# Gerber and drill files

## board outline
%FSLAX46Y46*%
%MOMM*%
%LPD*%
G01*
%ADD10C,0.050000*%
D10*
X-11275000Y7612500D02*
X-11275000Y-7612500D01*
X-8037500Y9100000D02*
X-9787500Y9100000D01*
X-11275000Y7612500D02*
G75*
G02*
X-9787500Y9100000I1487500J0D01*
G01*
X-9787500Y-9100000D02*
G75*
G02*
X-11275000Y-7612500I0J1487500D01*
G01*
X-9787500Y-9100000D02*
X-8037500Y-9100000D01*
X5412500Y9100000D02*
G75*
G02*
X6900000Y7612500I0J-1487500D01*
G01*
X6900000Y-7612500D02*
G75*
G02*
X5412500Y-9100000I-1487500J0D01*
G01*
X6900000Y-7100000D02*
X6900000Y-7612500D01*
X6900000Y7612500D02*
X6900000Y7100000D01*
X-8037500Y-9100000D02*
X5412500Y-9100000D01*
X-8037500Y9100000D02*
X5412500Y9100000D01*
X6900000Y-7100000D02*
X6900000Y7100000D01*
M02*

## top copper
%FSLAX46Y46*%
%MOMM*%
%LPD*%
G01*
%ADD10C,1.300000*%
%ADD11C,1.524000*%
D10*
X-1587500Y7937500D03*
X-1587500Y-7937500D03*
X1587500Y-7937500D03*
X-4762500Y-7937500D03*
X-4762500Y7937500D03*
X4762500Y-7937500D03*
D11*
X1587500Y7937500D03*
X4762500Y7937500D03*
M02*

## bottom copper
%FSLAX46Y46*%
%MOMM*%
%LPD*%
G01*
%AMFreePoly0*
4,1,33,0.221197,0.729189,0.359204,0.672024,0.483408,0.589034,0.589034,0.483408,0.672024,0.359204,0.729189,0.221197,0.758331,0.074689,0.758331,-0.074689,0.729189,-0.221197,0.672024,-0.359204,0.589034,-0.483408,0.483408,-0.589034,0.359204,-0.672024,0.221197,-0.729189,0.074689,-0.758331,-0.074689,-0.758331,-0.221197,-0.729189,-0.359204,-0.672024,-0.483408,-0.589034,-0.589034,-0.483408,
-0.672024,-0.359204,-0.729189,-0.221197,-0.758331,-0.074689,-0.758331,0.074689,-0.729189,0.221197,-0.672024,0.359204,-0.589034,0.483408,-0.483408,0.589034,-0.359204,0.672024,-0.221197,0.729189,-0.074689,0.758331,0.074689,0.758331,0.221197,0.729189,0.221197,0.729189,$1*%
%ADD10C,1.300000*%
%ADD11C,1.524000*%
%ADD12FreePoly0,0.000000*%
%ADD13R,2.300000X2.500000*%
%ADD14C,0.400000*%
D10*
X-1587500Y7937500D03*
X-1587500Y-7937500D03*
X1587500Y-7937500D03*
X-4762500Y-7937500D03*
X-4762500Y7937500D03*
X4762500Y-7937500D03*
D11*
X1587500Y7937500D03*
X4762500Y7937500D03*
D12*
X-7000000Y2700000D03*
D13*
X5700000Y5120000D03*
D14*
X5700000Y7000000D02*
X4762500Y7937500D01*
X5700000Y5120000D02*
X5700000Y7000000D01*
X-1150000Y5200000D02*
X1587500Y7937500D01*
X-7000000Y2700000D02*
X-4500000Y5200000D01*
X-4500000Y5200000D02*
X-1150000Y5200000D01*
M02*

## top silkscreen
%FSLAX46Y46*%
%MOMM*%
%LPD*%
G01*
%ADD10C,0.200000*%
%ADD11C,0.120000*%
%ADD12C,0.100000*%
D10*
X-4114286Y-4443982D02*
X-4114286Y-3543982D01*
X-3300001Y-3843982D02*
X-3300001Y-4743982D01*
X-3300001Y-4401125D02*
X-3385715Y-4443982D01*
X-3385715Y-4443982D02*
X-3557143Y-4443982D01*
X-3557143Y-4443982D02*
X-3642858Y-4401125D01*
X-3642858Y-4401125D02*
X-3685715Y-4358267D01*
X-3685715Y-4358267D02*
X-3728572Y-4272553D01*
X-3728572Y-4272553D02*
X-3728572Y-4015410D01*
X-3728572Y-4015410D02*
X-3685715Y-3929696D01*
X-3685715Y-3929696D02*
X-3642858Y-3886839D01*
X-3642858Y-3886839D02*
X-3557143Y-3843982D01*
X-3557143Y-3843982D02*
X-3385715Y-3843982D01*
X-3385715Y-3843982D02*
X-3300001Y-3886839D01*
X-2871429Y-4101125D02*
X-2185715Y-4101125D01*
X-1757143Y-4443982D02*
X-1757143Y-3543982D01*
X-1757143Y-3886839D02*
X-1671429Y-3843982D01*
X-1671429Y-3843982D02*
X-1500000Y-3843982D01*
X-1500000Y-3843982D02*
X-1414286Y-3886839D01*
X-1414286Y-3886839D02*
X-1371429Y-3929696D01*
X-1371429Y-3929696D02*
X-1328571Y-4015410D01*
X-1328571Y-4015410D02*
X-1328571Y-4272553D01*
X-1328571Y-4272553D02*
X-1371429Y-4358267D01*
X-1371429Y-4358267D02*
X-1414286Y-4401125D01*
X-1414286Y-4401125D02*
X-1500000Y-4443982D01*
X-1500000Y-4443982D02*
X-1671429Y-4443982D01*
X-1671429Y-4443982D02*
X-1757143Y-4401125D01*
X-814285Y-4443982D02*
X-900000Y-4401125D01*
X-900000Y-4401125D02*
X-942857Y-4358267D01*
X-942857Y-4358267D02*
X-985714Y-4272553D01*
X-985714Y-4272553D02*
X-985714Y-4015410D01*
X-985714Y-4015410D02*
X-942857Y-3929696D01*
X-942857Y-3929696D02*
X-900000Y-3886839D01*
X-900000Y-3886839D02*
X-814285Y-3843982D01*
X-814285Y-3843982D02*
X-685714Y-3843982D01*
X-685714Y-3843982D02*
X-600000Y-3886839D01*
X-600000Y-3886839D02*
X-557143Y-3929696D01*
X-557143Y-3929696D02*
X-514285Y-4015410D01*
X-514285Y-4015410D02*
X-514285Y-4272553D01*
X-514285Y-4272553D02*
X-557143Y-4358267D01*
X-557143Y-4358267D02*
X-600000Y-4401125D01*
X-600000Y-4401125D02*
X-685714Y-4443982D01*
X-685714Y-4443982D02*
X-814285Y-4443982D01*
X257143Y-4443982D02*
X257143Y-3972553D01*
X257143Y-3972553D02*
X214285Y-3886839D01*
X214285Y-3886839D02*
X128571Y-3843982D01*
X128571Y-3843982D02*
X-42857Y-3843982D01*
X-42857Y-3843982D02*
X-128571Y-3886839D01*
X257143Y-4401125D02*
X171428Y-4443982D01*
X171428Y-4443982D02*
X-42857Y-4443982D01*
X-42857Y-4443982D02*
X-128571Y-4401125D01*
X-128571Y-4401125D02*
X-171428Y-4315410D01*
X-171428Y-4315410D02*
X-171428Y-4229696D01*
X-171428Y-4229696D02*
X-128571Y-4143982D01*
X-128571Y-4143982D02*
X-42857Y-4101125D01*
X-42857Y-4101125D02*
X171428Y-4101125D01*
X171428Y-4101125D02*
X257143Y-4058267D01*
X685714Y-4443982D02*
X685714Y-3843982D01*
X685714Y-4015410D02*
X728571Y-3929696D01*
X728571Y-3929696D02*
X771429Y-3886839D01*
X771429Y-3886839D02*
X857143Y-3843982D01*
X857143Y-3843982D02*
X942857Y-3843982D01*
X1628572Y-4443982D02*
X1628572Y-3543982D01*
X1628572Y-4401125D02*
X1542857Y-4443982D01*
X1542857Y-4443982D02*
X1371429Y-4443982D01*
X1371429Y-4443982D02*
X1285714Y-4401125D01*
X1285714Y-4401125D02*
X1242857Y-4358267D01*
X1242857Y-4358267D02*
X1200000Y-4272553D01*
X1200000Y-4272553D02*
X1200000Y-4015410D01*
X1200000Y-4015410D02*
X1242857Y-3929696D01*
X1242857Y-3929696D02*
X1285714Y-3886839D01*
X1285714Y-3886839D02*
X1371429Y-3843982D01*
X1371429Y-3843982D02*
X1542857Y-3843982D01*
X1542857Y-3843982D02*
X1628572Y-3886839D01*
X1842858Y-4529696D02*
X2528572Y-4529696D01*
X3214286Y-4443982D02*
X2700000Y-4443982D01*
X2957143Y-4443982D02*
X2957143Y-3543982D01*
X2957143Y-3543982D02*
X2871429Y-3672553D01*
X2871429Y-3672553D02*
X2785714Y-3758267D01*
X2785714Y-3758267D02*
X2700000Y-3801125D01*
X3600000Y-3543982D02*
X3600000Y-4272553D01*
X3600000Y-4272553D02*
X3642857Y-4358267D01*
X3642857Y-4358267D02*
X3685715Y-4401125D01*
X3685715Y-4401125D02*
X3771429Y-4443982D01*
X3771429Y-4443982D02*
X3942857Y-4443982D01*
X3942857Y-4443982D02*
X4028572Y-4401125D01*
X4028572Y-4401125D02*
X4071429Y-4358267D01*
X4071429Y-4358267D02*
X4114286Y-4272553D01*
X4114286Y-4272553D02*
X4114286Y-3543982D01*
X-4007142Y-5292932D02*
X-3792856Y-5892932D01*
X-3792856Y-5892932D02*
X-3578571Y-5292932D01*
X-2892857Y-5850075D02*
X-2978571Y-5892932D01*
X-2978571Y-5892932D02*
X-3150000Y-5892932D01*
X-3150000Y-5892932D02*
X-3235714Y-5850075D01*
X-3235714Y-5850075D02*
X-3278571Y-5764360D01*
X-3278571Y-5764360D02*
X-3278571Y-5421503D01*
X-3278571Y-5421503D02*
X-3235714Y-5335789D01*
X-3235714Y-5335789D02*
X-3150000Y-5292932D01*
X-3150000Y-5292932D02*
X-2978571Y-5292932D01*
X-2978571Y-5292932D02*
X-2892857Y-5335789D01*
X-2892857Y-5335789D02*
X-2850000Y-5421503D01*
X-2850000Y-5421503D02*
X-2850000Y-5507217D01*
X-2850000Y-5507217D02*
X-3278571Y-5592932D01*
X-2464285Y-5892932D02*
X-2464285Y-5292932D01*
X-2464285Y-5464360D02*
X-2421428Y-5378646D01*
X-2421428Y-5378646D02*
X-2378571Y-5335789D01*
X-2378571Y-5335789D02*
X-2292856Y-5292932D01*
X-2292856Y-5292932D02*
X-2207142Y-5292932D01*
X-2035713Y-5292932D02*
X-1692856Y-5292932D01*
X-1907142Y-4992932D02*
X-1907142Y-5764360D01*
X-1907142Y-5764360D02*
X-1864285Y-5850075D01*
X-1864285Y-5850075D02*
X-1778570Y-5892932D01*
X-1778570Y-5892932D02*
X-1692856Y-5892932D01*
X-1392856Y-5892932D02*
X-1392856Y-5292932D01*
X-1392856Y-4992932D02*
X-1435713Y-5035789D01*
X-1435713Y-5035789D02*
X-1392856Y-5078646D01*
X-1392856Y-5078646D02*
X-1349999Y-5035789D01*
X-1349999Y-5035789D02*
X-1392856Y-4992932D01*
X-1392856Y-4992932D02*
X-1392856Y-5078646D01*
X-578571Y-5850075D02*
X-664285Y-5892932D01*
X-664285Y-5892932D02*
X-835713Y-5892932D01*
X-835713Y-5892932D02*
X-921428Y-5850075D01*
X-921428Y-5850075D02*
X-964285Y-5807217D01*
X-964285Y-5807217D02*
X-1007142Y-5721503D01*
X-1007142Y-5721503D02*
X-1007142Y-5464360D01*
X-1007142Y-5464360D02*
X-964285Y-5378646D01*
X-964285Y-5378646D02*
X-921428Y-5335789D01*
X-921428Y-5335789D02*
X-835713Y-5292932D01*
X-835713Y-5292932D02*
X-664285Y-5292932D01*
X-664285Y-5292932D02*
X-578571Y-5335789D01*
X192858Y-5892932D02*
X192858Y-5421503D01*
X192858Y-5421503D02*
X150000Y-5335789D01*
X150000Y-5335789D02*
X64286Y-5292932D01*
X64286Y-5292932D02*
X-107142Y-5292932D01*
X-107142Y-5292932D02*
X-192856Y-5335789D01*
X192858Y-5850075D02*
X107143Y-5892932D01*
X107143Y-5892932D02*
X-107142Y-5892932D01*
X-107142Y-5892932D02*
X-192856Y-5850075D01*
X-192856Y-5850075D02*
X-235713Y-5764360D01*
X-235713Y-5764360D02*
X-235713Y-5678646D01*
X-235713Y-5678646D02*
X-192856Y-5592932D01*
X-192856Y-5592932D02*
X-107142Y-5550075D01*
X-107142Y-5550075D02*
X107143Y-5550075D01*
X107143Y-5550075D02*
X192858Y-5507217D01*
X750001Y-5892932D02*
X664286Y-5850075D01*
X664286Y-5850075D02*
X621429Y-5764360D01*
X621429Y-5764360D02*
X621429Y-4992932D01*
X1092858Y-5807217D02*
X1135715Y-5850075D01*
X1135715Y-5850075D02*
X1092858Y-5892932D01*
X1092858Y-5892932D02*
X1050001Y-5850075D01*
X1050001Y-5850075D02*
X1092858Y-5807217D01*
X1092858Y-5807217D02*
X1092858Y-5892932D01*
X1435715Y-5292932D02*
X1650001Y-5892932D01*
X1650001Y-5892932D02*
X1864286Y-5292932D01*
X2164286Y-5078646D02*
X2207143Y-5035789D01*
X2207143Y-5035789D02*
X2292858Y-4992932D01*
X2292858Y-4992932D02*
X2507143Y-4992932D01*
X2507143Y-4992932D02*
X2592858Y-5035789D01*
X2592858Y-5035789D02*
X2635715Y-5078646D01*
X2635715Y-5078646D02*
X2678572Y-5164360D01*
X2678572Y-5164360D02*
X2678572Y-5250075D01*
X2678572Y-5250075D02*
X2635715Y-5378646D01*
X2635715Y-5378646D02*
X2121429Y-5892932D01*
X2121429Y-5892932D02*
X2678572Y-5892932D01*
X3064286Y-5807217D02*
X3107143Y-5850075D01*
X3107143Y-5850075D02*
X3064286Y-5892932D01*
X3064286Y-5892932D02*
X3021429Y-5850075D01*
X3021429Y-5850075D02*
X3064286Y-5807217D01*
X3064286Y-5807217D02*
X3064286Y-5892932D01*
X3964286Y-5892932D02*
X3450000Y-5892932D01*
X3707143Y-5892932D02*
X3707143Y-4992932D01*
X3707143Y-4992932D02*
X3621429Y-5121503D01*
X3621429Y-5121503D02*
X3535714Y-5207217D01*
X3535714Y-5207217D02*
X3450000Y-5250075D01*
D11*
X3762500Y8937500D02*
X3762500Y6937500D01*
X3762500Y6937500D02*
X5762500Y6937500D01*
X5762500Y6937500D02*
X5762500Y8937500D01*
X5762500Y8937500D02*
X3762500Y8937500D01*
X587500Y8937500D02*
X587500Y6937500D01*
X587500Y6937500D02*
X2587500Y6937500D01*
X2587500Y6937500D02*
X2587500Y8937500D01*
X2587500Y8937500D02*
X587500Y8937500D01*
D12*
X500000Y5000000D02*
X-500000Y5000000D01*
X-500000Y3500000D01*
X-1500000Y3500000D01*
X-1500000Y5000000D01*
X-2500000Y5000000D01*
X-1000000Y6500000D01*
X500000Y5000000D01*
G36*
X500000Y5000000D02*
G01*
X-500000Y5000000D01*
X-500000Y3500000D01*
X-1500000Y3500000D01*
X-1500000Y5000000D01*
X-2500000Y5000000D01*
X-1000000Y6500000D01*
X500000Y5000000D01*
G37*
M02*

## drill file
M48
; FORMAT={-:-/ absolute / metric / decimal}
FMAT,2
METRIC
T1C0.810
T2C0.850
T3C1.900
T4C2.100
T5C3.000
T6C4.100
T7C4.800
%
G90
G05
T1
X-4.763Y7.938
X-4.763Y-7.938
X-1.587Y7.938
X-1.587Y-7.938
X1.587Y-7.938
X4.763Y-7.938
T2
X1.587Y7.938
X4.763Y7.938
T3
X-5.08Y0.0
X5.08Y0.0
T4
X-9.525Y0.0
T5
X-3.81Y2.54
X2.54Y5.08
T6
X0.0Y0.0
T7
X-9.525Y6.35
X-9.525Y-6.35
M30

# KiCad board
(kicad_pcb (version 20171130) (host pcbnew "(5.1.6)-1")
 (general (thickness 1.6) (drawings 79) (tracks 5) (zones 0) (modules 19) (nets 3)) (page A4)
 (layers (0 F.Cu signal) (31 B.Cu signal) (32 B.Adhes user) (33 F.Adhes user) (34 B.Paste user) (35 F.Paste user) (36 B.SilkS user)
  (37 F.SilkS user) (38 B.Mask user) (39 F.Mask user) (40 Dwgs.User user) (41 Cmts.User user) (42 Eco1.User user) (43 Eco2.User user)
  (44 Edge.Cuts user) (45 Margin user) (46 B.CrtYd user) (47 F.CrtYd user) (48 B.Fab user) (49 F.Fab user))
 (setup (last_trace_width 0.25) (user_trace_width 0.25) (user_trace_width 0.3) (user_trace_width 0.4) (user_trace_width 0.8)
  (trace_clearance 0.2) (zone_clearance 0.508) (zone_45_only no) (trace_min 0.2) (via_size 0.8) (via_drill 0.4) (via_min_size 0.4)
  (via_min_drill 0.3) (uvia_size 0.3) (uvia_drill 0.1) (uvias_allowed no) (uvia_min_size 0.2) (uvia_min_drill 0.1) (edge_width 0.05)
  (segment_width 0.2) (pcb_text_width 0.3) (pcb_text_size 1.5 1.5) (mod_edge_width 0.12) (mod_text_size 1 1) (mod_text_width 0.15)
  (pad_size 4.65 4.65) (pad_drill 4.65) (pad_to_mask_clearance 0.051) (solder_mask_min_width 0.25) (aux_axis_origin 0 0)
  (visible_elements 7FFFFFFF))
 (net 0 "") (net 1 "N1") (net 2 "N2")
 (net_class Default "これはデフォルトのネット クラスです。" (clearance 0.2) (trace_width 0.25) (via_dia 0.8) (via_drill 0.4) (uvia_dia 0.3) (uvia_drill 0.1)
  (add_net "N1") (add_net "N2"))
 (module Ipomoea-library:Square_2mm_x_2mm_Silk (layer F.Cu) (at 4.7625 -7.9375)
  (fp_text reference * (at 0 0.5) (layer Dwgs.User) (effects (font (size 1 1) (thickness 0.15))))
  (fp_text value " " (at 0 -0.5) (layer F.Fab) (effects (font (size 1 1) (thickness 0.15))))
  (fp_line (start -1 -1) (end -1 1) (layer F.SilkS) (width 0.12))
  (fp_line (start -1 1) (end 1 1) (layer F.SilkS) (width 0.12))
  (fp_line (start 1 1) (end 1 -1) (layer F.SilkS) (width 0.12))
  (fp_line (start 1 -1) (end -1 -1) (layer F.SilkS) (width 0.12)))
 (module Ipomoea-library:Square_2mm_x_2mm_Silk (layer F.Cu) (at 1.5875 -7.9375)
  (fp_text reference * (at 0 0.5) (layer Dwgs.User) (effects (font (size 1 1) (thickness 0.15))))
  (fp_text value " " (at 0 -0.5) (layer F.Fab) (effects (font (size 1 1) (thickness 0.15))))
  (fp_line (start -1 -1) (end -1 1) (layer F.SilkS) (width 0.12))
  (fp_line (start -1 1) (end 1 1) (layer F.SilkS) (width 0.12))
  (fp_line (start 1 1) (end 1 -1) (layer F.SilkS) (width 0.12))
  (fp_line (start 1 -1) (end -1 -1) (layer F.SilkS) (width 0.12)))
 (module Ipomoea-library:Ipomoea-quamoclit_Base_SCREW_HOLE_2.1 (layer F.Cu) (at -9.525 0)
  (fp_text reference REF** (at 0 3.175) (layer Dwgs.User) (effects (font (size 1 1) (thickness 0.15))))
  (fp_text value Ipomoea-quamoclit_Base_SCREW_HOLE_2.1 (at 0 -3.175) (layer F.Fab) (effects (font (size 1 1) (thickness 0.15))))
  (pad "" np_thru_hole circle (at 0 0) (size 2.1 2.1) (drill 2.1) (layers *.Cu *.Mask)))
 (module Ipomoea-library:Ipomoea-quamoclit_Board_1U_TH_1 (layer F.Cu) (at -1.5875 -7.9375)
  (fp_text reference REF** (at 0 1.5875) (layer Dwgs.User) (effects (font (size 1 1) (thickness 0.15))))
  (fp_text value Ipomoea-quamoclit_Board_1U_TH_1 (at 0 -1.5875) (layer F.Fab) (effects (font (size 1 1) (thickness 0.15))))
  (pad "" thru_hole circle (at 0 0 180) (size 1.3 1.3) (drill 0.81) (layers *.Cu *.Mask)))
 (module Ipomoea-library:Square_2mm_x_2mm (layer F.Cu) (at -1.5875 -7.9375)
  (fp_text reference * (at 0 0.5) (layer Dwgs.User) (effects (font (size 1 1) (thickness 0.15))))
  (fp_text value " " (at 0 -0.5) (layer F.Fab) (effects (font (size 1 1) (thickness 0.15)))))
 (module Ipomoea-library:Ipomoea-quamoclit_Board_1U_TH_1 (layer F.Cu) (at -1.5875 7.9375)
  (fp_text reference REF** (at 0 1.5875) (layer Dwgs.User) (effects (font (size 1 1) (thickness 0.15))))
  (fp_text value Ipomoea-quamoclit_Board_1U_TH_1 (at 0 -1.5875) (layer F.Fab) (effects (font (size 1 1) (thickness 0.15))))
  (pad "" thru_hole circle (at 0 0 180) (size 1.3 1.3) (drill 0.81) (layers *.Cu *.Mask)))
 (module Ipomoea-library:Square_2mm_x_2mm (layer F.Cu) (at -1.5875 7.9375)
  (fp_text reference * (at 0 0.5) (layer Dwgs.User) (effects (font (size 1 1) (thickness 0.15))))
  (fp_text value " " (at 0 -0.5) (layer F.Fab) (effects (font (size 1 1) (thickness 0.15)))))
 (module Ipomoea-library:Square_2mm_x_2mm (layer F.Cu) (at 1.5875 7.9375)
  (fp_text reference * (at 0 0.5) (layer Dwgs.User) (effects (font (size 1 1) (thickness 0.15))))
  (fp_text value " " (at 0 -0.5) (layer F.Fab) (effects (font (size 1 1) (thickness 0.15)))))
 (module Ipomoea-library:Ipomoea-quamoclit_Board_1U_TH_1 (layer F.Cu) (at 1.5875 7.9375)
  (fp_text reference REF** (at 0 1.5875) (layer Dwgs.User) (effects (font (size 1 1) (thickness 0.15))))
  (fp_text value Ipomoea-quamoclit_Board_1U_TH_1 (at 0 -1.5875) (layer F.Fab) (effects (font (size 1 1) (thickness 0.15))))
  (pad "" thru_hole circle (at 0 0 180) (size 1.3 1.3) (drill 0.81) (layers *.Cu *.Mask)))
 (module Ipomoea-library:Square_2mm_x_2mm (layer F.Cu) (at 4.7625 7.9375)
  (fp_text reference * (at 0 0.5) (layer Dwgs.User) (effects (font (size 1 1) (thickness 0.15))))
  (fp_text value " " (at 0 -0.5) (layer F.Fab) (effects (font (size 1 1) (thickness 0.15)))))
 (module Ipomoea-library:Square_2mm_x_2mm (layer F.Cu) (at -4.7625 7.9375)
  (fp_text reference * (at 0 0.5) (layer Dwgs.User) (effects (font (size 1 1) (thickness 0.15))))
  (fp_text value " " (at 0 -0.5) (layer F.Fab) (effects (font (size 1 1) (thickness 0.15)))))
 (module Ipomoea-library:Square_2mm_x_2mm (layer F.Cu) (at -4.7625 -7.9375)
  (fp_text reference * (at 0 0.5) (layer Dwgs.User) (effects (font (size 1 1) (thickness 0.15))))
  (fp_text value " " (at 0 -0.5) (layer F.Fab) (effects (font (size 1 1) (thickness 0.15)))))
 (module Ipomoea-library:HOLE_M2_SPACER (layer F.Cu) (at -9.525 6.35)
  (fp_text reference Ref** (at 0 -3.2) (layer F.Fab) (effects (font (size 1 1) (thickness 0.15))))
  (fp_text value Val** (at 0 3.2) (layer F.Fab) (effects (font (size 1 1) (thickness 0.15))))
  (pad "" np_thru_hole circle (at 0 0) (size 4.8 4.8) (drill 4.8) (layers *.Cu *.Mask)))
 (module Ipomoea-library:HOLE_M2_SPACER (layer F.Cu) (at -9.525 -6.35)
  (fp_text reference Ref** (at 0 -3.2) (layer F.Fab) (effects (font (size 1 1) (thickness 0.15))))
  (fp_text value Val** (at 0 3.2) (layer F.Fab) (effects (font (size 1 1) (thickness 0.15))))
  (pad "" np_thru_hole circle (at 0 0) (size 4.8 4.8) (drill 4.8) (layers *.Cu *.Mask)))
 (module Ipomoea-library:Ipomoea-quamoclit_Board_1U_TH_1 (layer F.Cu) (at -4.7625 7.9375)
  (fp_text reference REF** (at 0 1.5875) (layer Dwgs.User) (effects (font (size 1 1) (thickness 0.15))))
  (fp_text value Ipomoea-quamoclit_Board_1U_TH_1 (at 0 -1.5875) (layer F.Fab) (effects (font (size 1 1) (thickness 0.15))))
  (pad "" thru_hole circle (at 0 0 180) (size 1.3 1.3) (drill 0.81) (layers *.Cu *.Mask)))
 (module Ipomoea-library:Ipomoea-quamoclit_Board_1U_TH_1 (layer F.Cu) (at -4.7625 -7.9375)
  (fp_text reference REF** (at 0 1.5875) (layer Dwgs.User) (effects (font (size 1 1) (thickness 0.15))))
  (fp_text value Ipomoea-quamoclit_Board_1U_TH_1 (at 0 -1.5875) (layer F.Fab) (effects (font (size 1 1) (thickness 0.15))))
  (pad "" thru_hole circle (at 0 0 180) (size 1.3 1.3) (drill 0.81) (layers *.Cu *.Mask)))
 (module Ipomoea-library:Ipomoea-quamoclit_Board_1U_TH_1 (layer F.Cu) (at 4.7625 7.9375)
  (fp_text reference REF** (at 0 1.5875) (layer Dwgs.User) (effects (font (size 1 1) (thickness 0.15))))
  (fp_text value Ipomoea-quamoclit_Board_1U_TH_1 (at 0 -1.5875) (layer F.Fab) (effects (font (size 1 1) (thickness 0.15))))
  (pad "" thru_hole circle (at 0 0 180) (size 1.3 1.3) (drill 0.81) (layers *.Cu *.Mask)))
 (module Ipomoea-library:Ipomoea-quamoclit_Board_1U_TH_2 (layer F.Cu) (at 3.175 -7.9375)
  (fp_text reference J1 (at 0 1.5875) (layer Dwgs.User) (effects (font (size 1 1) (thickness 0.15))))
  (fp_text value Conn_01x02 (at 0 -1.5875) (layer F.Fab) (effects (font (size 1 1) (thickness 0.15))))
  (pad 1 thru_hole circle (at -1.5875 0 180) (size 1.524 1.524) (drill 0.85) (layers *.Cu *.Mask) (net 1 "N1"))
  (pad 2 thru_hole circle (at 1.5875 0 180) (size 1.524 1.524) (drill 0.85) (layers *.Cu *.Mask) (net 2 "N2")))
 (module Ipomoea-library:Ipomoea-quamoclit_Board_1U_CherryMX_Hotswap (layer F.Cu) (at 0 0)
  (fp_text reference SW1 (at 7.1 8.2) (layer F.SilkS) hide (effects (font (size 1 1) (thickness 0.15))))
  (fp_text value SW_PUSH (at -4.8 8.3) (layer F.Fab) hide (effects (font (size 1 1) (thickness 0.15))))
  (fp_poly (pts (xy 0.5 -5) (xy -0.5 -5) (xy -0.5 -3.5) (xy -1.5 -3.5) (xy -1.5 -5) (xy -2.5 -5) (xy -1 -6.5)) (layer F.SilkS) (width 0.1))
  (pad "" np_thru_hole circle (at 0 0 90) (size 4.1 4.1) (drill 4.1) (layers *.Cu *.Mask))
  (pad "" np_thru_hole circle (at 5.08 0) (size 1.9 1.9) (drill 1.9) (layers *.Cu *.Mask))
  (pad "" np_thru_hole circle (at -5.08 0) (size 1.9 1.9) (drill 1.9) (layers *.Cu *.Mask))
  (pad 1 smd custom (at -7 -2.7) (size 1.524 1.524) (layers B.Cu B.Paste B.Mask) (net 1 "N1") (zone_connect 0)
   (options (clearance outline) (anchor circle)) (primitives))
  (pad "" np_thru_hole circle (at 2.54 -5.08 180) (size 3 3) (drill 3) (layers *.Cu *.Mask))
  (pad 2 smd rect (at 5.7 -5.12 180) (size 2.3 2.5) (layers B.Cu B.Paste B.Mask) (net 2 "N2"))
  (pad "" np_thru_hole circle (at -3.81 -2.54 180) (size 3 3) (drill 3) (layers *.Cu *.Mask)))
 (gr_line (start -11.275 -7.6125) (end -11.275 7.6125) (layer Edge.Cuts) (width 0.05))
 (gr_line (start -8.0375 -9.1) (end -9.7875 -9.1) (layer Edge.Cuts) (width 0.05))
 (gr_arc (start -9.7875 -7.6125) (end -9.7875 -9.1) (angle -90) (layer Edge.Cuts) (width 0.05))
 (gr_arc (start -9.7875 7.6125) (end -11.275 7.6125) (angle -90) (layer Edge.Cuts) (width 0.05))
 (gr_line (start -9.7875 9.1) (end -8.0375 9.1) (layer Edge.Cuts) (width 0.05))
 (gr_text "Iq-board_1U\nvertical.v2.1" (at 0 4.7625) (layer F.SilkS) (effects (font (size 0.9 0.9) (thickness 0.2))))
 (gr_arc (start 5.4125 -7.6125) (end 6.9 -7.6125) (angle -90) (layer Edge.Cuts) (width 0.05))
 (gr_arc (start 5.4125 7.6125) (end 5.4125 9.1) (angle -90) (layer Edge.Cuts) (width 0.05))
 (gr_line (start 6.9 7.1) (end 6.9 7.6125) (layer Edge.Cuts) (width 0.05))
 (gr_line (start 6.9 -7.6125) (end 6.9 -7.1) (layer Edge.Cuts) (width 0.05))
 (gr_line (start -8.0375 9.1) (end 5.4125 9.1) (layer Edge.Cuts) (width 0.05))
 (gr_line (start -8.0375 -9.1) (end 5.4125 -9.1) (layer Edge.Cuts) (width 0.05))
 (gr_line (start 6.9 7.1) (end 6.9 -7.1) (layer Edge.Cuts) (width 0.05))
 (segment (start 5.7 -7) (end 4.7625 -7.9375) (width 0.4) (layer B.Cu) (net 2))
 (segment (start 5.7 -5.12) (end 5.7 -7) (width 0.4) (layer B.Cu) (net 2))
 (segment (start -1.15 -5.2) (end 1.5875 -7.9375) (width 0.4) (layer B.Cu) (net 1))
 (segment (start -7 -2.7) (end -4.5 -5.2) (width 0.4) (layer B.Cu) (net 1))
 (segment (start -4.5 -5.2) (end -1.15 -5.2) (width 0.4) (layer B.Cu) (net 1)))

